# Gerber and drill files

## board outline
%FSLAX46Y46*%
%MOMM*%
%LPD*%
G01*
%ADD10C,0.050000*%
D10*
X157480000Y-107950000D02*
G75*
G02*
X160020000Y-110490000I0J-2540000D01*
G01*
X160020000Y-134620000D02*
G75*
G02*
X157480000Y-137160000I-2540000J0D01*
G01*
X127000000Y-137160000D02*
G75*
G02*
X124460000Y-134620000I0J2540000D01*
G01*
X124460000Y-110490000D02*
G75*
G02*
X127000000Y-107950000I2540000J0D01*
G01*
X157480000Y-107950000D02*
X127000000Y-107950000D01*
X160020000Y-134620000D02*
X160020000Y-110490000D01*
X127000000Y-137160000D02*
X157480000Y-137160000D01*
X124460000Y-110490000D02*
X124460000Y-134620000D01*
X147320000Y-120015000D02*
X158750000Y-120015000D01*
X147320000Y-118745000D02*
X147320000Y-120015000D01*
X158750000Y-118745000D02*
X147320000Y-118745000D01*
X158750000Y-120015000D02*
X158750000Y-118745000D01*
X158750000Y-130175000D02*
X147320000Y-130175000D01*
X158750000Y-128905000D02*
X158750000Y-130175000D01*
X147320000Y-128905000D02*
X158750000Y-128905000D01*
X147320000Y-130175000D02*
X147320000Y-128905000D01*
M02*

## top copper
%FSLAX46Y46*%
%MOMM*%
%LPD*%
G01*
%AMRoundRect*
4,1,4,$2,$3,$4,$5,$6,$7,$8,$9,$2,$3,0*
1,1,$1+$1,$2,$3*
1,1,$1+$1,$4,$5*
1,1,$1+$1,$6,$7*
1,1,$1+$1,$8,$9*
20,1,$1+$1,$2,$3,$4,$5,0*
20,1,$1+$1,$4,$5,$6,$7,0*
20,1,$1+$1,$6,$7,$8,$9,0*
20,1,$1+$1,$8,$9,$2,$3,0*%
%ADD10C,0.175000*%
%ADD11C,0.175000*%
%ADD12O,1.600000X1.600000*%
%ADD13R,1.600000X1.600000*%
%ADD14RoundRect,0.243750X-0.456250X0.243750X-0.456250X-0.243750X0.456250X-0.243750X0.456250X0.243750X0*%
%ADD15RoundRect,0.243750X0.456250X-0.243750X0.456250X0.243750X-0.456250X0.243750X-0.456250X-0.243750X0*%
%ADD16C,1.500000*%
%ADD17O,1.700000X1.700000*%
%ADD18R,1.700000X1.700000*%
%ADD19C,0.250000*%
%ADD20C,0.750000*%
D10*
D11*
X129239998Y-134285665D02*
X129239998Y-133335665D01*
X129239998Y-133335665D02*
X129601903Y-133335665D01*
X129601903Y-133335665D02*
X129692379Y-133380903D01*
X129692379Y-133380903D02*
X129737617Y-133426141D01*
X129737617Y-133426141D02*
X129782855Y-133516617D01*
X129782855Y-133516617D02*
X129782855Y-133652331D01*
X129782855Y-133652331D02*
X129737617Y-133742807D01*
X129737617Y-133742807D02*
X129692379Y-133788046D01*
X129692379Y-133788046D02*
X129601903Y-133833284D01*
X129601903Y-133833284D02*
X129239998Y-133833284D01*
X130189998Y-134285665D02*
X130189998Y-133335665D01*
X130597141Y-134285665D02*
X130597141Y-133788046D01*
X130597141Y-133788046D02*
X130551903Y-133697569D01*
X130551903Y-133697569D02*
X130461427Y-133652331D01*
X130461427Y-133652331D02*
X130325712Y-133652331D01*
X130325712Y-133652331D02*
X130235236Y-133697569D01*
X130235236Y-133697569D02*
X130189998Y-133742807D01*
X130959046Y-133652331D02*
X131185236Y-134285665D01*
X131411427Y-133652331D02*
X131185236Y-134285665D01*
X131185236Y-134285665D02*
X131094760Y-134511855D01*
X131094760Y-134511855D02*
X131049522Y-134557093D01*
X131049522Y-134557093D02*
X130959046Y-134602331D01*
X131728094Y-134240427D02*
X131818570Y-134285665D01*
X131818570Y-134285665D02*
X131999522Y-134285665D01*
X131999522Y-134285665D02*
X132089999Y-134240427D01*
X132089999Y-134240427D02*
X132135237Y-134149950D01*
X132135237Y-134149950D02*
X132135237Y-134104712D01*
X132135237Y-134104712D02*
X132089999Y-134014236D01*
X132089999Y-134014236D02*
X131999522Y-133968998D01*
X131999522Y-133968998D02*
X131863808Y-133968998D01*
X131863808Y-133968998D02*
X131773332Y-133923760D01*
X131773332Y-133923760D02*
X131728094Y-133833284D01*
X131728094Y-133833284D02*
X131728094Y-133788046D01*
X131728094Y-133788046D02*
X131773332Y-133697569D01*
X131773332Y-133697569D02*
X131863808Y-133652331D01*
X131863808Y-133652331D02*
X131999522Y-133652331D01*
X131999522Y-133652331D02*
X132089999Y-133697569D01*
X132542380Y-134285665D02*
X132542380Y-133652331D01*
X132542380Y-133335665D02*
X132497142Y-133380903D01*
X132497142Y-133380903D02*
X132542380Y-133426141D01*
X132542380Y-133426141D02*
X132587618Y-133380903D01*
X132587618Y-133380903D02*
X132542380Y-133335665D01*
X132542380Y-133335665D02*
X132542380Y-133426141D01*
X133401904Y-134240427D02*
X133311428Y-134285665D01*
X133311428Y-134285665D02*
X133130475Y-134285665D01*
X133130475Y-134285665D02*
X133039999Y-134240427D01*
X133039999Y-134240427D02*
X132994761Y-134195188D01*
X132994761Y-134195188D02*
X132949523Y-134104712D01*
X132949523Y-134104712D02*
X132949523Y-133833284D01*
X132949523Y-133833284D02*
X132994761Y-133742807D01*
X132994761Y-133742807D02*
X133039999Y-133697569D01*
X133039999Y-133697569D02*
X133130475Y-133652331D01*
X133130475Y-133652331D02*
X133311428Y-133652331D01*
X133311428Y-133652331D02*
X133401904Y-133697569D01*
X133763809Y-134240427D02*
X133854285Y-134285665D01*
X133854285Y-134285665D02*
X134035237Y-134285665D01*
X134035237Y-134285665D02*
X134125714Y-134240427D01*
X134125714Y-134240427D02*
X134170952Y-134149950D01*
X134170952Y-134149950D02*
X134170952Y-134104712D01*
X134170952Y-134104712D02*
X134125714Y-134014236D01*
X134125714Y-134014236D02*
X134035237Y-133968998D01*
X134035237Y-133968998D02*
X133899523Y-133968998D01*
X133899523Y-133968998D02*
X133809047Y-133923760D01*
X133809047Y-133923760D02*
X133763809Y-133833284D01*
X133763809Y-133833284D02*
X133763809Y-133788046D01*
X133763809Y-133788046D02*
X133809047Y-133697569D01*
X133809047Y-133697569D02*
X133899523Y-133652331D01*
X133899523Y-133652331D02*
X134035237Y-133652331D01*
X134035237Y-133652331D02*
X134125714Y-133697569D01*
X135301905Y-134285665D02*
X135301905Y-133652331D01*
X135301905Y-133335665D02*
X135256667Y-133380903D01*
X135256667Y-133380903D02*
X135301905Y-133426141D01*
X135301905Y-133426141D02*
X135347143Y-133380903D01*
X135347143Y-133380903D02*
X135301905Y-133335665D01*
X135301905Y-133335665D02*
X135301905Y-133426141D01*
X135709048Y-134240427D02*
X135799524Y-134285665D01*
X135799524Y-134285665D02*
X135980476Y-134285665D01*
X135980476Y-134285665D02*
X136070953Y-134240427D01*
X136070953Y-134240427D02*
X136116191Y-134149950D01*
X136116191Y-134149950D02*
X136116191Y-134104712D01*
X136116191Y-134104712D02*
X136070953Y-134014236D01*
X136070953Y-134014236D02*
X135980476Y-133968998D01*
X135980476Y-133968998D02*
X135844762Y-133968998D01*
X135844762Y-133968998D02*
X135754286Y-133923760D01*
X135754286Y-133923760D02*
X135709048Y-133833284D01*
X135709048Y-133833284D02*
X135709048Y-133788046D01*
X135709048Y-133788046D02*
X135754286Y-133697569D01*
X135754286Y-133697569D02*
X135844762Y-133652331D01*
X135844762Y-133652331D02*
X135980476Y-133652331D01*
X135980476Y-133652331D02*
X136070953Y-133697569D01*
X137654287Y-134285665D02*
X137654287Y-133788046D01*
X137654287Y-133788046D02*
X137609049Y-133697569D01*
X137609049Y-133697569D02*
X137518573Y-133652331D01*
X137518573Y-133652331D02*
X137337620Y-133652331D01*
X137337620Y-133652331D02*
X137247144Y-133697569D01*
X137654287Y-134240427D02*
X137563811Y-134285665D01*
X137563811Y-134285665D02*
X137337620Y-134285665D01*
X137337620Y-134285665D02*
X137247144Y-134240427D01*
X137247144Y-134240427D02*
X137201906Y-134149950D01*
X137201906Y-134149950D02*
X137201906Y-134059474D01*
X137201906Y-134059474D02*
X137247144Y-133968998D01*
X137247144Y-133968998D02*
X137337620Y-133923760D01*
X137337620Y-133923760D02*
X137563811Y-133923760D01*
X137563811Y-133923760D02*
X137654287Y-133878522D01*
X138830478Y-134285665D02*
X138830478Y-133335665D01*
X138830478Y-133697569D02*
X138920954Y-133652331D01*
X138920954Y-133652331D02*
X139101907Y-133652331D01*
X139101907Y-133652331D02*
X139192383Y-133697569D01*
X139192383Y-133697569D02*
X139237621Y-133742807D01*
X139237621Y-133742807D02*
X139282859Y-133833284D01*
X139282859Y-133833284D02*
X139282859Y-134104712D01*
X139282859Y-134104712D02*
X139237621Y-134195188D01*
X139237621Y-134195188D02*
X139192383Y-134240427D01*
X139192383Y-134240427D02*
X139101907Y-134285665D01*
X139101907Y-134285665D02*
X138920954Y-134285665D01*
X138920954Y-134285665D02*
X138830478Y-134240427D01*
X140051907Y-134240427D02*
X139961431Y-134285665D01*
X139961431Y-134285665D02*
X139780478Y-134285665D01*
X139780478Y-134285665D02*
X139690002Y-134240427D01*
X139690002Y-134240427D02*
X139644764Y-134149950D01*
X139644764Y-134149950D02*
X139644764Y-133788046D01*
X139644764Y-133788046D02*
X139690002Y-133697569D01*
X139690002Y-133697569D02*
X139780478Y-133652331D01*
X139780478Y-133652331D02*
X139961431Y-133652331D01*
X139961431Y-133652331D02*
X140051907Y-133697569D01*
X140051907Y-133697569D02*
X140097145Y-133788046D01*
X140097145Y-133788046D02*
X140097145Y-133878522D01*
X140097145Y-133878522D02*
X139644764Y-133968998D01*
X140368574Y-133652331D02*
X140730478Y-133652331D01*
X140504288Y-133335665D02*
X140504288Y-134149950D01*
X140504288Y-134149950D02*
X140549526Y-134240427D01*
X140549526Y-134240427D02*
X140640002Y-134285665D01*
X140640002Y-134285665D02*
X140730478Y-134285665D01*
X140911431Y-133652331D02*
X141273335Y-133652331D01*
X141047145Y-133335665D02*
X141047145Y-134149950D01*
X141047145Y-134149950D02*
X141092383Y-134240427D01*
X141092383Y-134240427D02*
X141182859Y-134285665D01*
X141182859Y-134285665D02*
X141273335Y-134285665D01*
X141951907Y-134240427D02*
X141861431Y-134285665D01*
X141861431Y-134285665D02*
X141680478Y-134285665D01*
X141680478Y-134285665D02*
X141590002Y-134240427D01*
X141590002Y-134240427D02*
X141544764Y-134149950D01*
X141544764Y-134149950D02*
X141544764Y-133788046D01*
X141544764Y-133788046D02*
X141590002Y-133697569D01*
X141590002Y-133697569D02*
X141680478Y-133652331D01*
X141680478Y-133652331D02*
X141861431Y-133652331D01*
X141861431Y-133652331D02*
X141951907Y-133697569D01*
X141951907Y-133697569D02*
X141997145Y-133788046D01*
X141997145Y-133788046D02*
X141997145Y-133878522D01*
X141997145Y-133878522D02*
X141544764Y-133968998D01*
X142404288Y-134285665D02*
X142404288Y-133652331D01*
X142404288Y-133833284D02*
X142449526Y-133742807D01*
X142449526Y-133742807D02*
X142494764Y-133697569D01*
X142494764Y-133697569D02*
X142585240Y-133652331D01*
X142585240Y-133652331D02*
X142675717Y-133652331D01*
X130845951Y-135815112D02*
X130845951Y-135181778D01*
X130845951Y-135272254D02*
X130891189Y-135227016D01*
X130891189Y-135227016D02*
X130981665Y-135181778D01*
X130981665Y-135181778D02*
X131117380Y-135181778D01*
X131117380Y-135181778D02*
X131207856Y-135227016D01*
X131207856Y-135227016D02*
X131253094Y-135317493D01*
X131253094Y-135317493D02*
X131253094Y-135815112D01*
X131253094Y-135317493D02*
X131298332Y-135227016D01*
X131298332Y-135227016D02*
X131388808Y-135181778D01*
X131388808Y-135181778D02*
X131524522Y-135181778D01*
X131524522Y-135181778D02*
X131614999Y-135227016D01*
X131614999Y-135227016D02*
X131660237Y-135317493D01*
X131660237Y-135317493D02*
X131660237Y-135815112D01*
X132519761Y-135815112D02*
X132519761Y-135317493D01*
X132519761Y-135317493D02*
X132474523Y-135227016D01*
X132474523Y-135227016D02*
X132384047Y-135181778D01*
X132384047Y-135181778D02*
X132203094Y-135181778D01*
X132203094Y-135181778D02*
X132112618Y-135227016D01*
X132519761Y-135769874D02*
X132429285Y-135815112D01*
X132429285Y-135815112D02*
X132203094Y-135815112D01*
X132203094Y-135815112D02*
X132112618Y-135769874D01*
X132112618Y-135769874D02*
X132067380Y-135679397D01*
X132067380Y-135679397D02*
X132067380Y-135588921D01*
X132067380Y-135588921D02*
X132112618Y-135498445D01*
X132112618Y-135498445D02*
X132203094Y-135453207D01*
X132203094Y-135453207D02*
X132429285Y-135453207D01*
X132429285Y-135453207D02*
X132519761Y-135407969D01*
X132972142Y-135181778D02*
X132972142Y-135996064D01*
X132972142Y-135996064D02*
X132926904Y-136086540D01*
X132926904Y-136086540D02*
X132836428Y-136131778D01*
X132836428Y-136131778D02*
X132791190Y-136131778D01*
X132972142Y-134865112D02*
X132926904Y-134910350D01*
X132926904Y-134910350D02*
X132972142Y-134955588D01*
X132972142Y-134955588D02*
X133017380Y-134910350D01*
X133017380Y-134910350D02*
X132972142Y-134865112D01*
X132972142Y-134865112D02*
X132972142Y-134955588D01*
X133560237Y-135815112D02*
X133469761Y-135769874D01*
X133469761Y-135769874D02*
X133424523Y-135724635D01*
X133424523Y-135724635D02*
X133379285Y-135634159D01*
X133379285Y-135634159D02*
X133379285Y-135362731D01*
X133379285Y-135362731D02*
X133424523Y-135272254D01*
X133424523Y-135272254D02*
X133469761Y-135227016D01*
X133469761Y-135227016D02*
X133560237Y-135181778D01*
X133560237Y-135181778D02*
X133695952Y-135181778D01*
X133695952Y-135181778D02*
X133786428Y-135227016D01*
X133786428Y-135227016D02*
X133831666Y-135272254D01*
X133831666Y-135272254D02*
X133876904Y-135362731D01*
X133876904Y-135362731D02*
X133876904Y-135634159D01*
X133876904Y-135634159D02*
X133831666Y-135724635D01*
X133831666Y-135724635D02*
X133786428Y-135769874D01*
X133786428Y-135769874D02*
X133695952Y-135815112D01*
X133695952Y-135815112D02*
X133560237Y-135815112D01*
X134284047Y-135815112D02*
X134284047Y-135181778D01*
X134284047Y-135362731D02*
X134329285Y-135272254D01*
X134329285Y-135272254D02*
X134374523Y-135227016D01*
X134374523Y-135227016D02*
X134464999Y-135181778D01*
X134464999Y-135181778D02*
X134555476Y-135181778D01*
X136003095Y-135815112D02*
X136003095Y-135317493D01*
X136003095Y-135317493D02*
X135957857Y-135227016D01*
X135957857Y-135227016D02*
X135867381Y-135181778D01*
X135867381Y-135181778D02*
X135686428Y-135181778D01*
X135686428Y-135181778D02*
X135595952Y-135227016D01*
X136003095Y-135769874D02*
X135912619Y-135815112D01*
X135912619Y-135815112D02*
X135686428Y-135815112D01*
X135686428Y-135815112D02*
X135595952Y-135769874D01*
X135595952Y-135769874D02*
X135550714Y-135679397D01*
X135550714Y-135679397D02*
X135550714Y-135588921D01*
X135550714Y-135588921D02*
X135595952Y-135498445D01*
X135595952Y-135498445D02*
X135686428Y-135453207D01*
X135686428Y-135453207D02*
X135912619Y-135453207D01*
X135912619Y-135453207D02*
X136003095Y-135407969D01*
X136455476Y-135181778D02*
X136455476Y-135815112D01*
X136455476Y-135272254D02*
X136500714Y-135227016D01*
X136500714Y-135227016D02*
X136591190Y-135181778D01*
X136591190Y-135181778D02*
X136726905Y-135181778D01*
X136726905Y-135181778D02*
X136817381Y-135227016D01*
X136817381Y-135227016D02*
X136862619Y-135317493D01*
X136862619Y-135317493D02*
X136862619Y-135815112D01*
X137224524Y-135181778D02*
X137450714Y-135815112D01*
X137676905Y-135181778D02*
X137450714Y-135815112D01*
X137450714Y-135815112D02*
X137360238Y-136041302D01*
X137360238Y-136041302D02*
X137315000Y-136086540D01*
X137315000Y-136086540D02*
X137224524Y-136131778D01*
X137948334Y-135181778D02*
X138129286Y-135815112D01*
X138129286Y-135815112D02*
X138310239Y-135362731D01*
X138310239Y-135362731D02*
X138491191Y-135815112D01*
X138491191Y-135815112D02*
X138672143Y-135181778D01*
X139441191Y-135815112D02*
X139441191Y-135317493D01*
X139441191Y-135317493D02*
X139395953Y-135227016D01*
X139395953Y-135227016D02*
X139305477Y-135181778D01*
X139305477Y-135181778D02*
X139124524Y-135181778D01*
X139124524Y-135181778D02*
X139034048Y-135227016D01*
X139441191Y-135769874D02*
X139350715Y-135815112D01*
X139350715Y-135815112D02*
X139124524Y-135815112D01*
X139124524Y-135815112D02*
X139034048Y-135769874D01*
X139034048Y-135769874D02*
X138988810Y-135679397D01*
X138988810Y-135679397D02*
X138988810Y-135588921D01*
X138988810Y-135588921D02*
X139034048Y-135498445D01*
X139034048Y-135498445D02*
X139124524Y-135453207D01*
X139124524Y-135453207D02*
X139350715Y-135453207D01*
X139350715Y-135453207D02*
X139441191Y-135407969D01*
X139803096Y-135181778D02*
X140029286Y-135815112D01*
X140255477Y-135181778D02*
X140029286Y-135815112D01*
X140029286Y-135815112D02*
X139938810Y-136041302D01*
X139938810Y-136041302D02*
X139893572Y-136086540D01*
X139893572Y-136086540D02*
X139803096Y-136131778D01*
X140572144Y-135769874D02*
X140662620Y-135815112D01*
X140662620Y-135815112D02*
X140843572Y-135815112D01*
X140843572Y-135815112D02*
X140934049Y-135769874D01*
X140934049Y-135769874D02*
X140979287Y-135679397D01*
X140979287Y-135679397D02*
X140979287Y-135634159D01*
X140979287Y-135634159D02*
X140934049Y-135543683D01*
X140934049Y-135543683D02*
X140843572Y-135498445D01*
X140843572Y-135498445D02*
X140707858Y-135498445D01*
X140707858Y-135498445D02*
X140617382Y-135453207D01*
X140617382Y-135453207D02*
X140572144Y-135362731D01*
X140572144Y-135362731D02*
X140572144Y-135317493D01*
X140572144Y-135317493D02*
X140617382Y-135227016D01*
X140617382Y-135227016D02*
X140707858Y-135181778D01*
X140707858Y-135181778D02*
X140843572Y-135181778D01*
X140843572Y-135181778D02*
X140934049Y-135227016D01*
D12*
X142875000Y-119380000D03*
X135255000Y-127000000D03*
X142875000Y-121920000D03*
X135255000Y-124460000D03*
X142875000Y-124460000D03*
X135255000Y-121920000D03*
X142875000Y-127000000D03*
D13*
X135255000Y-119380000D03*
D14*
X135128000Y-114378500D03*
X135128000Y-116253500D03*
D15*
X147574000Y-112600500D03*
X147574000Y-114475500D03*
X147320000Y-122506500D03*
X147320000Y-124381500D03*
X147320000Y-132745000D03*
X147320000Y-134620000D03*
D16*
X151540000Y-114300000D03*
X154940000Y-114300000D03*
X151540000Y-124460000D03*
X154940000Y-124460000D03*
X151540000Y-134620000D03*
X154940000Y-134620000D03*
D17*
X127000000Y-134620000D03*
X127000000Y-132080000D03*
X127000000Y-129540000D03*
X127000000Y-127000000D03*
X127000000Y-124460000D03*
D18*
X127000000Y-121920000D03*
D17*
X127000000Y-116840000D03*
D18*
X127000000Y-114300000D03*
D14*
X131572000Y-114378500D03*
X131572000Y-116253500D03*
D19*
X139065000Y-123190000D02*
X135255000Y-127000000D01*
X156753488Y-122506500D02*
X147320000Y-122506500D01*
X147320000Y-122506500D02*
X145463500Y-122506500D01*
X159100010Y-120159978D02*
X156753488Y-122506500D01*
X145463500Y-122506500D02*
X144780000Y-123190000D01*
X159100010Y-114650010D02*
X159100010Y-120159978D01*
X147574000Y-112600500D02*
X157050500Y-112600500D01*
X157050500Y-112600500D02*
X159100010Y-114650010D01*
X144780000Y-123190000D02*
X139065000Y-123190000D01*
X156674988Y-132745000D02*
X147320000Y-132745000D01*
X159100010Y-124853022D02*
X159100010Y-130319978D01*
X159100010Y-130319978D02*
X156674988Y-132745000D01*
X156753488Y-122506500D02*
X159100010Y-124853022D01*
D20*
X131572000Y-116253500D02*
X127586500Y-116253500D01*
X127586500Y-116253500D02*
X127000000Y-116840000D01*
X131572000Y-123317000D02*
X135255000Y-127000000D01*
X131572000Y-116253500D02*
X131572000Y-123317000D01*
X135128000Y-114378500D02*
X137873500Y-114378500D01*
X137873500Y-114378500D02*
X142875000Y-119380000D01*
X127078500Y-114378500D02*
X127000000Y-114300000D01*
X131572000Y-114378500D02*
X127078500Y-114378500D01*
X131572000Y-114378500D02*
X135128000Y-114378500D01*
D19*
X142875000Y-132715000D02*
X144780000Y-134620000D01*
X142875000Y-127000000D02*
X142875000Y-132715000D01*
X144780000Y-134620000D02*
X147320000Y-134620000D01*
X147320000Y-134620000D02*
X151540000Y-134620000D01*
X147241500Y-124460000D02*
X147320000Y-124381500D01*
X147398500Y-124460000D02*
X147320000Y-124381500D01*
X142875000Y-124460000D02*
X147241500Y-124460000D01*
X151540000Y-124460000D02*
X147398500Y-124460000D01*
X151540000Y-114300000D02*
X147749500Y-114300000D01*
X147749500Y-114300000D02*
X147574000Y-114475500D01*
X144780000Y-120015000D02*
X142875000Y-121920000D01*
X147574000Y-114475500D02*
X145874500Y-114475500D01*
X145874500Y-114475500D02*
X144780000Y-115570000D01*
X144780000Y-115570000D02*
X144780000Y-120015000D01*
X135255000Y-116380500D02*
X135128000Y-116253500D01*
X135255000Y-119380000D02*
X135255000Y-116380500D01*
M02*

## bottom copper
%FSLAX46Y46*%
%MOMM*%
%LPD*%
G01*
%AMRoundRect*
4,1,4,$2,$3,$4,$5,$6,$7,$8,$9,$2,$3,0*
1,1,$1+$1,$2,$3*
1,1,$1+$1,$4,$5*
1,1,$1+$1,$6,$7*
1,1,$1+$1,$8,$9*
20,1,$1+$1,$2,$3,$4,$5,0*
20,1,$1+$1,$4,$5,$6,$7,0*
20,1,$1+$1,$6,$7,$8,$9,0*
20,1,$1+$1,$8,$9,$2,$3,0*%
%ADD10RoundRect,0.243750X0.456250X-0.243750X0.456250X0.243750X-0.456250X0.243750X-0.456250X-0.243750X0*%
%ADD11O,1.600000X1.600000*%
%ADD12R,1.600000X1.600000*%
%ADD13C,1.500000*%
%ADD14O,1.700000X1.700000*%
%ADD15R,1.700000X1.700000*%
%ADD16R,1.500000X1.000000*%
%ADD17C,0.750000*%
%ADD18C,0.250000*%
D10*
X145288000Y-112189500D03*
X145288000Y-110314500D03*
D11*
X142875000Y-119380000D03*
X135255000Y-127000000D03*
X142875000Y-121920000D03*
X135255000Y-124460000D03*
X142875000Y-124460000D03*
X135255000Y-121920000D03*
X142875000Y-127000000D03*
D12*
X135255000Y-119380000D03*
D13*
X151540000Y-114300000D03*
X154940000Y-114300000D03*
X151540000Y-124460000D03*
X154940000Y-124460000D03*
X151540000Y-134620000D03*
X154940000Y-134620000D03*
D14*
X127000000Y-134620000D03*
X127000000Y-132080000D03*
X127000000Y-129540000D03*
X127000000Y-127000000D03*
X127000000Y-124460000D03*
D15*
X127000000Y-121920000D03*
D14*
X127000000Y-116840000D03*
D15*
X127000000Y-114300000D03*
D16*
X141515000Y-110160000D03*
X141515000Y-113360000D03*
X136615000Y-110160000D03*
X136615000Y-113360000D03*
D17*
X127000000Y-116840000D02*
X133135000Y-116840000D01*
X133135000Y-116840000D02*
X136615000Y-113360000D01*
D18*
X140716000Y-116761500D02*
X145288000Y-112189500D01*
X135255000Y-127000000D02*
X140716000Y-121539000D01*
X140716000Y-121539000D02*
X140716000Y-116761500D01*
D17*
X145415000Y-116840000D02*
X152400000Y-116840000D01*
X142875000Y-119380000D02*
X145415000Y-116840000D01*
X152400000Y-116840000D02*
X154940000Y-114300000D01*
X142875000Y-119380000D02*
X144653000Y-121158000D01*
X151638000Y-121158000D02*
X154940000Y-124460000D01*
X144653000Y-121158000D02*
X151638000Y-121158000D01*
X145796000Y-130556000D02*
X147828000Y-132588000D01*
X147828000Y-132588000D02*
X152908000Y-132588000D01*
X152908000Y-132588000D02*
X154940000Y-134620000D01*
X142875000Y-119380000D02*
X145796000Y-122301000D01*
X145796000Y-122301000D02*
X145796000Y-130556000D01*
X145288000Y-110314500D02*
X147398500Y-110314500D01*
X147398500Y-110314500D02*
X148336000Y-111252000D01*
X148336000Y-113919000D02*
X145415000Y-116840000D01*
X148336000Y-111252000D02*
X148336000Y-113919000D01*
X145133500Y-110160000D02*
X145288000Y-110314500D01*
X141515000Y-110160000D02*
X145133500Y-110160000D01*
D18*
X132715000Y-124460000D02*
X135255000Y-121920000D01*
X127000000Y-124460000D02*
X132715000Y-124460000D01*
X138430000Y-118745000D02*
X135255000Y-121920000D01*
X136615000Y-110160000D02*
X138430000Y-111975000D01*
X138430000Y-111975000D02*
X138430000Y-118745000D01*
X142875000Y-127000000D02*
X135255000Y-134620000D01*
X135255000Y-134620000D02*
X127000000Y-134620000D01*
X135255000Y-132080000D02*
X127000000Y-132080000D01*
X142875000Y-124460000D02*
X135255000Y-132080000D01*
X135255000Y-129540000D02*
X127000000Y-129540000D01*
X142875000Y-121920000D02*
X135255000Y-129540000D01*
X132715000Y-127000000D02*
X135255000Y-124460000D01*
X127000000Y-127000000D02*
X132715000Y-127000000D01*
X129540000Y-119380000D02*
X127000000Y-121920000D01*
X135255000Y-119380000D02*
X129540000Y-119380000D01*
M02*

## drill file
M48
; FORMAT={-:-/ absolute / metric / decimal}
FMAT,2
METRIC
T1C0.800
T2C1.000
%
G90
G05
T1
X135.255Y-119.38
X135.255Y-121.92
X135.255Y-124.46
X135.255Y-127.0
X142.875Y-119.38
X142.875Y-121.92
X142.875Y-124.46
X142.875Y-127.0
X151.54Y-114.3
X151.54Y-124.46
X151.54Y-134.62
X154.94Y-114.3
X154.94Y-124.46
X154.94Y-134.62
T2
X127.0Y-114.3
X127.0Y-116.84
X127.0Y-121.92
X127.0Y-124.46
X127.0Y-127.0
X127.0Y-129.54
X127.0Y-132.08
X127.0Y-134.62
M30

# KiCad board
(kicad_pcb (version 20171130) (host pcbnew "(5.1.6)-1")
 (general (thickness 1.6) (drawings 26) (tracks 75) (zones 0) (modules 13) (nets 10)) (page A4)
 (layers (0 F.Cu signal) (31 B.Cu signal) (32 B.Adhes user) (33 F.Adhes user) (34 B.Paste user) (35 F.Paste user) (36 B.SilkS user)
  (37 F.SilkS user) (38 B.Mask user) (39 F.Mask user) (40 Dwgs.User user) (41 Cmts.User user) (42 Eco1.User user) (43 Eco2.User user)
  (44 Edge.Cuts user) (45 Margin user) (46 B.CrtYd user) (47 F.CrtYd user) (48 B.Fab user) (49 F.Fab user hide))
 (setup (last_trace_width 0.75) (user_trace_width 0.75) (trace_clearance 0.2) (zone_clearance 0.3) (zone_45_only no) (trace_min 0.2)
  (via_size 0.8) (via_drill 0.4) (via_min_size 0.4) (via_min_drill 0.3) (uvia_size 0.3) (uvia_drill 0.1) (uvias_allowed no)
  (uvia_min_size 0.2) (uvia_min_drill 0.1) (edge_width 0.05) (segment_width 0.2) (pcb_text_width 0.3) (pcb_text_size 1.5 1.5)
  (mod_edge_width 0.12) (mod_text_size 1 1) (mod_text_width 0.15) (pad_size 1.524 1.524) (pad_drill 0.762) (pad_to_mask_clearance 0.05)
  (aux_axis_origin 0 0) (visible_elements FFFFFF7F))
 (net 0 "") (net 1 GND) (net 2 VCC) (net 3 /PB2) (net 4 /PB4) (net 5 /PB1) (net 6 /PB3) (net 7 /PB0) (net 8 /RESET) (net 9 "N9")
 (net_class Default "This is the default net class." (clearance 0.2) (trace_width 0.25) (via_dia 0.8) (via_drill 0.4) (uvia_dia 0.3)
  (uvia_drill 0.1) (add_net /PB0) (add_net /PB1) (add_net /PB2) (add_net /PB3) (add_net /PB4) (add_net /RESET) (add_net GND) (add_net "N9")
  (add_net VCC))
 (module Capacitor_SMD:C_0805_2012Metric (layer B.Cu) (at 145.288 111.252 90)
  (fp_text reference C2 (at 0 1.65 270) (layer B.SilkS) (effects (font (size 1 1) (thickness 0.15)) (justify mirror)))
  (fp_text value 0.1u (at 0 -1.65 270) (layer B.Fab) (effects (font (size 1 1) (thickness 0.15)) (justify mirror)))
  (pad 1 smd roundrect (at -0.9375 0 90) (size 0.975 1.4) (layers B.Cu B.Paste B.Mask) (roundrect_rratio 0.25) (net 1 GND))
  (pad 2 smd roundrect (at 0.9375 0 90) (size 0.975 1.4) (layers B.Cu B.Paste B.Mask) (roundrect_rratio 0.25) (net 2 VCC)))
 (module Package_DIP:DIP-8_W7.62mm (layer F.Cu) (at 135.255 119.38)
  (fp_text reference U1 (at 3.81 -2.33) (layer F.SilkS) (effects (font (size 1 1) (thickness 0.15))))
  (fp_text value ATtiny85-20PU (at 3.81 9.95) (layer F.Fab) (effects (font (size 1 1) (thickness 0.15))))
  (pad 8 thru_hole oval (at 7.62 0) (size 1.6 1.6) (drill 0.8) (layers *.Cu *.Mask) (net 2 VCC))
  (pad 4 thru_hole oval (at 0 7.62) (size 1.6 1.6) (drill 0.8) (layers *.Cu *.Mask) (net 1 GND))
  (pad 7 thru_hole oval (at 7.62 2.54) (size 1.6 1.6) (drill 0.8) (layers *.Cu *.Mask) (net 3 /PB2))
  (pad 3 thru_hole oval (at 0 5.08) (size 1.6 1.6) (drill 0.8) (layers *.Cu *.Mask) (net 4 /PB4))
  (pad 6 thru_hole oval (at 7.62 5.08) (size 1.6 1.6) (drill 0.8) (layers *.Cu *.Mask) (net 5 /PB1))
  (pad 2 thru_hole oval (at 0 2.54) (size 1.6 1.6) (drill 0.8) (layers *.Cu *.Mask) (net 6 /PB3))
  (pad 5 thru_hole oval (at 7.62 7.62) (size 1.6 1.6) (drill 0.8) (layers *.Cu *.Mask) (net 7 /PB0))
  (pad 1 thru_hole rect (at 0 0) (size 1.6 1.6) (drill 0.8) (layers *.Cu *.Mask) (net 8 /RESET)))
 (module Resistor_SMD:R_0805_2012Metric (layer F.Cu) (at 135.128 115.316 270)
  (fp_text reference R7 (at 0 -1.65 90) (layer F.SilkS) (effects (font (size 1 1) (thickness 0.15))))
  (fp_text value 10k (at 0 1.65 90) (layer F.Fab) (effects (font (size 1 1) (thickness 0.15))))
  (pad 1 smd roundrect (at -0.9375 0 270) (size 0.975 1.4) (layers F.Cu F.Paste F.Mask) (roundrect_rratio 0.25) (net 2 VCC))
  (pad 2 smd roundrect (at 0.9375 0 270) (size 0.975 1.4) (layers F.Cu F.Paste F.Mask) (roundrect_rratio 0.25) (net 8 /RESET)))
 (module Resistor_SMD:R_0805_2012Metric (layer F.Cu) (at 147.574 113.538 90)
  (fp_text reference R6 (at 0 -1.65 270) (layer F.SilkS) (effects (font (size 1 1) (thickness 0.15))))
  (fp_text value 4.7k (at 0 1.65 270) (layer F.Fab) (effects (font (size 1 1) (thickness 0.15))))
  (pad 2 smd roundrect (at 0.9375 0 90) (size 0.975 1.4) (layers F.Cu F.Paste F.Mask) (roundrect_rratio 0.25) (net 1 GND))
  (pad 1 smd roundrect (at -0.9375 0 90) (size 0.975 1.4) (layers F.Cu F.Paste F.Mask) (roundrect_rratio 0.25) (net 3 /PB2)))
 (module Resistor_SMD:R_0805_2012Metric (layer F.Cu) (at 147.32 123.444 90)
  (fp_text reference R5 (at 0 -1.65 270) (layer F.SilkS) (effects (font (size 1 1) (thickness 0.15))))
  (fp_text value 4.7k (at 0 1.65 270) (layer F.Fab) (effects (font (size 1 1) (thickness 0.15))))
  (pad 2 smd roundrect (at 0.9375 0 90) (size 0.975 1.4) (layers F.Cu F.Paste F.Mask) (roundrect_rratio 0.25) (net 1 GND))
  (pad 1 smd roundrect (at -0.9375 0 90) (size 0.975 1.4) (layers F.Cu F.Paste F.Mask) (roundrect_rratio 0.25) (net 5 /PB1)))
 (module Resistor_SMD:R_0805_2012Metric (layer F.Cu) (at 147.32 133.6825 90)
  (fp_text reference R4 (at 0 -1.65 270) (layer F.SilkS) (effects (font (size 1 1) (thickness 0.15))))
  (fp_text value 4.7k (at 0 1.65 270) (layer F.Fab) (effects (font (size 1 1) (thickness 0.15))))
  (pad 2 smd roundrect (at 0.9375 0 90) (size 0.975 1.4) (layers F.Cu F.Paste F.Mask) (roundrect_rratio 0.25) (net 1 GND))
  (pad 1 smd roundrect (at -0.9375 0 90) (size 0.975 1.4) (layers F.Cu F.Paste F.Mask) (roundrect_rratio 0.25) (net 7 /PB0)))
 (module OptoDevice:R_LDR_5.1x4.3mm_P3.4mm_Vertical (layer F.Cu) (at 154.94 114.3 180)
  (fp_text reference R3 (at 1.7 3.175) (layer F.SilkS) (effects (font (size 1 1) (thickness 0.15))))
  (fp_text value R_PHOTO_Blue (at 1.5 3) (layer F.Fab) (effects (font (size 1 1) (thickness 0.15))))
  (pad 2 thru_hole circle (at 3.4 0 180) (size 1.5 1.5) (drill 0.8) (layers *.Cu *.Mask) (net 3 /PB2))
  (pad 1 thru_hole circle (at 0 0 180) (size 1.5 1.5) (drill 0.8) (layers *.Cu *.Mask) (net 2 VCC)))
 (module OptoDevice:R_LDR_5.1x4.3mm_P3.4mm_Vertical (layer F.Cu) (at 154.94 124.46 180)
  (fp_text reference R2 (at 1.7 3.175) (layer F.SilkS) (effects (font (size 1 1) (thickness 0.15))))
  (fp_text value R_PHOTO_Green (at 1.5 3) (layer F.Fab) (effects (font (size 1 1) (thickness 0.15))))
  (pad 2 thru_hole circle (at 3.4 0 180) (size 1.5 1.5) (drill 0.8) (layers *.Cu *.Mask) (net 5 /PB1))
  (pad 1 thru_hole circle (at 0 0 180) (size 1.5 1.5) (drill 0.8) (layers *.Cu *.Mask) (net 2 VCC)))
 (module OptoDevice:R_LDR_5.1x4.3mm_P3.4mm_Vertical (layer F.Cu) (at 154.94 134.62 180)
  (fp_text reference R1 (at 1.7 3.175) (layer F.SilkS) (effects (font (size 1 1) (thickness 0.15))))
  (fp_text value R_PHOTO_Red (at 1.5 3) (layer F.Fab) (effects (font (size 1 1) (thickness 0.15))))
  (pad 2 thru_hole circle (at 3.4 0 180) (size 1.5 1.5) (drill 0.8) (layers *.Cu *.Mask) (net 7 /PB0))
  (pad 1 thru_hole circle (at 0 0 180) (size 1.5 1.5) (drill 0.8) (layers *.Cu *.Mask) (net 2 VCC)))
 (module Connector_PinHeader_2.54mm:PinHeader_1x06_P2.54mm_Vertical (layer F.Cu) (at 127 121.92)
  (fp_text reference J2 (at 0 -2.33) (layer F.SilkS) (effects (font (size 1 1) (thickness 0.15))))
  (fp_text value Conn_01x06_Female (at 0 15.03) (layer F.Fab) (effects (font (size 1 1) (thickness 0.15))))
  (pad 6 thru_hole oval (at 0 12.7) (size 1.7 1.7) (drill 1) (layers *.Cu *.Mask) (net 7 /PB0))
  (pad 5 thru_hole oval (at 0 10.16) (size 1.7 1.7) (drill 1) (layers *.Cu *.Mask) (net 5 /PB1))
  (pad 4 thru_hole oval (at 0 7.62) (size 1.7 1.7) (drill 1) (layers *.Cu *.Mask) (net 3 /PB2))
  (pad 3 thru_hole oval (at 0 5.08) (size 1.7 1.7) (drill 1) (layers *.Cu *.Mask) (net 4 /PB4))
  (pad 2 thru_hole oval (at 0 2.54) (size 1.7 1.7) (drill 1) (layers *.Cu *.Mask) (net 6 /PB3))
  (pad 1 thru_hole rect (at 0 0) (size 1.7 1.7) (drill 1) (layers *.Cu *.Mask) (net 8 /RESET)))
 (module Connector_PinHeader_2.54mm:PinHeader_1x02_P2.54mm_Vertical (layer F.Cu) (at 127 114.3)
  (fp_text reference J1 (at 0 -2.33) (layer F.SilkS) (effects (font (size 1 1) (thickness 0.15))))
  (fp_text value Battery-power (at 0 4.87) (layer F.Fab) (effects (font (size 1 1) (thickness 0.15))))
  (pad 2 thru_hole oval (at 0 2.54) (size 1.7 1.7) (drill 1) (layers *.Cu *.Mask) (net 1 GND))
  (pad 1 thru_hole rect (at 0 0) (size 1.7 1.7) (drill 1) (layers *.Cu *.Mask) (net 2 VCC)))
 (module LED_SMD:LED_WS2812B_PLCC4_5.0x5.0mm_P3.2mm (layer B.Cu) (at 139.065 111.76 180)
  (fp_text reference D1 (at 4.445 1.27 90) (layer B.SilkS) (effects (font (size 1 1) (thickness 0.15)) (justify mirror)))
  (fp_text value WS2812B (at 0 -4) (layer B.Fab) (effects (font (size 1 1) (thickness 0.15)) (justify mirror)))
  (pad 1 smd rect (at -2.45 1.6 180) (size 1.5 1) (layers B.Cu B.Paste B.Mask) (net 2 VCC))
  (pad 2 smd rect (at -2.45 -1.6 180) (size 1.5 1) (layers B.Cu B.Paste B.Mask) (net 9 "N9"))
  (pad 4 smd rect (at 2.45 1.6 180) (size 1.5 1) (layers B.Cu B.Paste B.Mask) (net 6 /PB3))
  (pad 3 smd rect (at 2.45 -1.6 180) (size 1.5 1) (layers B.Cu B.Paste B.Mask) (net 1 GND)))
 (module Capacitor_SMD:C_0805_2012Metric (layer F.Cu) (at 131.572 115.316 270)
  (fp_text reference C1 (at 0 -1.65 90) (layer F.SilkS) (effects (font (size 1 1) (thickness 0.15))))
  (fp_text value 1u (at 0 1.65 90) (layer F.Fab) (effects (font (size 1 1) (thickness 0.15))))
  (pad 1 smd roundrect (at -0.9375 0 270) (size 0.975 1.4) (layers F.Cu F.Paste F.Mask) (roundrect_rratio 0.25) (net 2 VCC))
  (pad 2 smd roundrect (at 0.9375 0 270) (size 0.975 1.4) (layers F.Cu F.Paste F.Mask) (roundrect_rratio 0.25) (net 1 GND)))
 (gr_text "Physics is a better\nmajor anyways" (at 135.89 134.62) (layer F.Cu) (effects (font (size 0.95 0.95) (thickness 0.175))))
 (gr_arc (start 157.48 110.49) (end 160.02 110.49) (angle -90) (layer Edge.Cuts) (width 0.05))
 (gr_arc (start 157.48 134.62) (end 157.48 137.16) (angle -90) (layer Edge.Cuts) (width 0.05))
 (gr_arc (start 127 134.62) (end 124.46 134.62) (angle -90) (layer Edge.Cuts) (width 0.05))
 (gr_arc (start 127 110.49) (end 127 107.95) (angle -90) (layer Edge.Cuts) (width 0.05))
 (gr_line (start 157.48 107.95) (end 127 107.95) (layer Edge.Cuts) (width 0.05))
 (gr_line (start 160.02 134.62) (end 160.02 110.49) (layer Edge.Cuts) (width 0.05))
 (gr_line (start 127 137.16) (end 157.48 137.16) (layer Edge.Cuts) (width 0.05))
 (gr_line (start 124.46 110.49) (end 124.46 134.62) (layer Edge.Cuts) (width 0.05))
 (gr_line (start 147.32 120.015) (end 158.75 120.015) (layer Edge.Cuts) (width 0.05))
 (gr_line (start 147.32 118.745) (end 147.32 120.015) (layer Edge.Cuts) (width 0.05))
 (gr_line (start 158.75 118.745) (end 147.32 118.745) (layer Edge.Cuts) (width 0.05))
 (gr_line (start 158.75 120.015) (end 158.75 118.745) (layer Edge.Cuts) (width 0.05))
 (gr_line (start 158.75 130.175) (end 147.32 130.175) (layer Edge.Cuts) (width 0.05))
 (gr_line (start 158.75 128.905) (end 158.75 130.175) (layer Edge.Cuts) (width 0.05))
 (gr_line (start 147.32 128.905) (end 158.75 128.905) (layer Edge.Cuts) (width 0.05))
 (gr_line (start 147.32 130.175) (end 147.32 128.905) (layer Edge.Cuts) (width 0.05))
 (segment (start 139.065 123.19) (end 135.255 127) (width 0.25) (layer F.Cu) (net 1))
 (segment (start 156.753488 122.5065) (end 147.32 122.5065) (width 0.25) (layer F.Cu) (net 1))
 (segment (start 147.32 122.5065) (end 145.4635 122.5065) (width 0.25) (layer F.Cu) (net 1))
 (segment (start 159.10001 120.159978) (end 156.753488 122.5065) (width 0.25) (layer F.Cu) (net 1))
 (segment (start 145.4635 122.5065) (end 144.78 123.19) (width 0.25) (layer F.Cu) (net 1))
 (segment (start 159.10001 114.65001) (end 159.10001 120.159978) (width 0.25) (layer F.Cu) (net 1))
 (segment (start 147.574 112.6005) (end 157.0505 112.6005) (width 0.25) (layer F.Cu) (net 1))
 (segment (start 157.0505 112.6005) (end 159.10001 114.65001) (width 0.25) (layer F.Cu) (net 1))
 (segment (start 144.78 123.19) (end 139.065 123.19) (width 0.25) (layer F.Cu) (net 1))
 (segment (start 156.674988 132.745) (end 147.32 132.745) (width 0.25) (layer F.Cu) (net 1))
 (segment (start 159.10001 124.853022) (end 159.10001 130.319978) (width 0.25) (layer F.Cu) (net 1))
 (segment (start 159.10001 130.319978) (end 156.674988 132.745) (width 0.25) (layer F.Cu) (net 1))
 (segment (start 156.753488 122.5065) (end 159.10001 124.853022) (width 0.25) (layer F.Cu) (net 1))
 (segment (start 131.572 116.2535) (end 127.5865 116.2535) (width 0.75) (layer F.Cu) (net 1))
 (segment (start 127.5865 116.2535) (end 127 116.84) (width 0.75) (layer F.Cu) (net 1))
 (segment (start 127 116.84) (end 133.135 116.84) (width 0.75) (layer B.Cu) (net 1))
 (segment (start 131.572 123.317) (end 135.255 127) (width 0.75) (layer F.Cu) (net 1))
 (segment (start 131.572 116.2535) (end 131.572 123.317) (width 0.75) (layer F.Cu) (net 1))
 (segment (start 133.135 116.84) (end 136.615 113.36) (width 0.75) (layer B.Cu) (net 1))
 (segment (start 140.716 116.7615) (end 145.288 112.1895) (width 0.25) (layer B.Cu) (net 1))
 (segment (start 135.255 127) (end 140.716 121.539) (width 0.25) (layer B.Cu) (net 1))
 (segment (start 140.716 121.539) (end 140.716 116.7615) (width 0.25) (layer B.Cu) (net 1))
 (segment (start 145.415 116.84) (end 152.4 116.84) (width 0.75) (layer B.Cu) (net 2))
 (segment (start 142.875 119.38) (end 145.415 116.84) (width 0.75) (layer B.Cu) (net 2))
 (segment (start 152.4 116.84) (end 154.94 114.3) (width 0.75) (layer B.Cu) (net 2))
 (segment (start 135.128 114.3785) (end 137.8735 114.3785) (width 0.75) (layer F.Cu) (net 2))
 (segment (start 137.8735 114.3785) (end 142.875 119.38) (width 0.75) (layer F.Cu) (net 2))
 (segment (start 127.0785 114.3785) (end 127 114.3) (width 0.75) (layer F.Cu) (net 2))
 (segment (start 131.572 114.3785) (end 127.0785 114.3785) (width 0.75) (layer F.Cu) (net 2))
 (segment (start 131.572 114.3785) (end 135.128 114.3785) (width 0.75) (layer F.Cu) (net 2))
 (segment (start 142.875 119.38) (end 144.653 121.158) (width 0.75) (layer B.Cu) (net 2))
 (segment (start 151.638 121.158) (end 154.94 124.46) (width 0.75) (layer B.Cu) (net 2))
 (segment (start 144.653 121.158) (end 151.638 121.158) (width 0.75) (layer B.Cu) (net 2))
 (segment (start 145.796 130.556) (end 147.828 132.588) (width 0.75) (layer B.Cu) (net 2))
 (segment (start 147.828 132.588) (end 152.908 132.588) (width 0.75) (layer B.Cu) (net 2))
 (segment (start 152.908 132.588) (end 154.94 134.62) (width 0.75) (layer B.Cu) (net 2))
 (segment (start 142.875 119.38) (end 145.796 122.301) (width 0.75) (layer B.Cu) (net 2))
 (segment (start 145.796 122.301) (end 145.796 130.556) (width 0.75) (layer B.Cu) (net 2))
 (segment (start 145.288 110.3145) (end 147.3985 110.3145) (width 0.75) (layer B.Cu) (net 2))
 (segment (start 147.3985 110.3145) (end 148.336 111.252) (width 0.75) (layer B.Cu) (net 2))
 (segment (start 148.336 113.919) (end 145.415 116.84) (width 0.75) (layer B.Cu) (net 2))
 (segment (start 148.336 111.252) (end 148.336 113.919) (width 0.75) (layer B.Cu) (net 2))
 (segment (start 145.1335 110.16) (end 145.288 110.3145) (width 0.75) (layer B.Cu) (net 2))
 (segment (start 141.515 110.16) (end 145.1335 110.16) (width 0.75) (layer B.Cu) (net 2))
 (segment (start 132.715 124.46) (end 135.255 121.92) (width 0.25) (layer B.Cu) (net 6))
 (segment (start 127 124.46) (end 132.715 124.46) (width 0.25) (layer B.Cu) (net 6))
 (segment (start 138.43 118.745) (end 135.255 121.92) (width 0.25) (layer B.Cu) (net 6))
 (segment (start 136.615 110.16) (end 138.43 111.975) (width 0.25) (layer B.Cu) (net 6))
 (segment (start 138.43 111.975) (end 138.43 118.745) (width 0.25) (layer B.Cu) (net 6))
 (segment (start 142.875 127) (end 135.255 134.62) (width 0.25) (layer B.Cu) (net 7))
 (segment (start 135.255 134.62) (end 127 134.62) (width 0.25) (layer B.Cu) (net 7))
 (segment (start 142.875 132.715) (end 144.78 134.62) (width 0.25) (layer F.Cu) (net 7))
 (segment (start 142.875 127) (end 142.875 132.715) (width 0.25) (layer F.Cu) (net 7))
 (segment (start 144.78 134.62) (end 147.32 134.62) (width 0.25) (layer F.Cu) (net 7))
 (segment (start 147.32 134.62) (end 151.54 134.62) (width 0.25) (layer F.Cu) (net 7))
 (segment (start 135.255 132.08) (end 127 132.08) (width 0.25) (layer B.Cu) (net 5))
 (segment (start 142.875 124.46) (end 135.255 132.08) (width 0.25) (layer B.Cu) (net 5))
 (segment (start 147.2415 124.46) (end 147.32 124.3815) (width 0.25) (layer F.Cu) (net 5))
 (segment (start 147.3985 124.46) (end 147.32 124.3815) (width 0.25) (layer F.Cu) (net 5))
 (segment (start 142.875 124.46) (end 147.2415 124.46) (width 0.25) (layer F.Cu) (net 5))
 (segment (start 151.54 124.46) (end 147.3985 124.46) (width 0.25) (layer F.Cu) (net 5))
 (segment (start 135.255 129.54) (end 127 129.54) (width 0.25) (layer B.Cu) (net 3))
 (segment (start 142.875 121.92) (end 135.255 129.54) (width 0.25) (layer B.Cu) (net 3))
 (segment (start 151.54 114.3) (end 147.7495 114.3) (width 0.25) (layer F.Cu) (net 3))
 (segment (start 147.7495 114.3) (end 147.574 114.4755) (width 0.25) (layer F.Cu) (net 3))
 (segment (start 144.78 120.015) (end 142.875 121.92) (width 0.25) (layer F.Cu) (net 3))
 (segment (start 147.574 114.4755) (end 145.8745 114.4755) (width 0.25) (layer F.Cu) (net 3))
 (segment (start 145.8745 114.4755) (end 144.78 115.57) (width 0.25) (layer F.Cu) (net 3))
 (segment (start 144.78 115.57) (end 144.78 120.015) (width 0.25) (layer F.Cu) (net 3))
 (segment (start 132.715 127) (end 135.255 124.46) (width 0.25) (layer B.Cu) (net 4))
 (segment (start 127 127) (end 132.715 127) (width 0.25) (layer B.Cu) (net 4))
 (segment (start 129.54 119.38) (end 127 121.92) (width 0.25) (layer B.Cu) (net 8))
 (segment (start 135.255 119.38) (end 129.54 119.38) (width 0.25) (layer B.Cu) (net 8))
 (segment (start 135.255 116.3805) (end 135.128 116.2535) (width 0.25) (layer F.Cu) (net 8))
 (segment (start 135.255 119.38) (end 135.255 116.3805) (width 0.25) (layer F.Cu) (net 8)))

